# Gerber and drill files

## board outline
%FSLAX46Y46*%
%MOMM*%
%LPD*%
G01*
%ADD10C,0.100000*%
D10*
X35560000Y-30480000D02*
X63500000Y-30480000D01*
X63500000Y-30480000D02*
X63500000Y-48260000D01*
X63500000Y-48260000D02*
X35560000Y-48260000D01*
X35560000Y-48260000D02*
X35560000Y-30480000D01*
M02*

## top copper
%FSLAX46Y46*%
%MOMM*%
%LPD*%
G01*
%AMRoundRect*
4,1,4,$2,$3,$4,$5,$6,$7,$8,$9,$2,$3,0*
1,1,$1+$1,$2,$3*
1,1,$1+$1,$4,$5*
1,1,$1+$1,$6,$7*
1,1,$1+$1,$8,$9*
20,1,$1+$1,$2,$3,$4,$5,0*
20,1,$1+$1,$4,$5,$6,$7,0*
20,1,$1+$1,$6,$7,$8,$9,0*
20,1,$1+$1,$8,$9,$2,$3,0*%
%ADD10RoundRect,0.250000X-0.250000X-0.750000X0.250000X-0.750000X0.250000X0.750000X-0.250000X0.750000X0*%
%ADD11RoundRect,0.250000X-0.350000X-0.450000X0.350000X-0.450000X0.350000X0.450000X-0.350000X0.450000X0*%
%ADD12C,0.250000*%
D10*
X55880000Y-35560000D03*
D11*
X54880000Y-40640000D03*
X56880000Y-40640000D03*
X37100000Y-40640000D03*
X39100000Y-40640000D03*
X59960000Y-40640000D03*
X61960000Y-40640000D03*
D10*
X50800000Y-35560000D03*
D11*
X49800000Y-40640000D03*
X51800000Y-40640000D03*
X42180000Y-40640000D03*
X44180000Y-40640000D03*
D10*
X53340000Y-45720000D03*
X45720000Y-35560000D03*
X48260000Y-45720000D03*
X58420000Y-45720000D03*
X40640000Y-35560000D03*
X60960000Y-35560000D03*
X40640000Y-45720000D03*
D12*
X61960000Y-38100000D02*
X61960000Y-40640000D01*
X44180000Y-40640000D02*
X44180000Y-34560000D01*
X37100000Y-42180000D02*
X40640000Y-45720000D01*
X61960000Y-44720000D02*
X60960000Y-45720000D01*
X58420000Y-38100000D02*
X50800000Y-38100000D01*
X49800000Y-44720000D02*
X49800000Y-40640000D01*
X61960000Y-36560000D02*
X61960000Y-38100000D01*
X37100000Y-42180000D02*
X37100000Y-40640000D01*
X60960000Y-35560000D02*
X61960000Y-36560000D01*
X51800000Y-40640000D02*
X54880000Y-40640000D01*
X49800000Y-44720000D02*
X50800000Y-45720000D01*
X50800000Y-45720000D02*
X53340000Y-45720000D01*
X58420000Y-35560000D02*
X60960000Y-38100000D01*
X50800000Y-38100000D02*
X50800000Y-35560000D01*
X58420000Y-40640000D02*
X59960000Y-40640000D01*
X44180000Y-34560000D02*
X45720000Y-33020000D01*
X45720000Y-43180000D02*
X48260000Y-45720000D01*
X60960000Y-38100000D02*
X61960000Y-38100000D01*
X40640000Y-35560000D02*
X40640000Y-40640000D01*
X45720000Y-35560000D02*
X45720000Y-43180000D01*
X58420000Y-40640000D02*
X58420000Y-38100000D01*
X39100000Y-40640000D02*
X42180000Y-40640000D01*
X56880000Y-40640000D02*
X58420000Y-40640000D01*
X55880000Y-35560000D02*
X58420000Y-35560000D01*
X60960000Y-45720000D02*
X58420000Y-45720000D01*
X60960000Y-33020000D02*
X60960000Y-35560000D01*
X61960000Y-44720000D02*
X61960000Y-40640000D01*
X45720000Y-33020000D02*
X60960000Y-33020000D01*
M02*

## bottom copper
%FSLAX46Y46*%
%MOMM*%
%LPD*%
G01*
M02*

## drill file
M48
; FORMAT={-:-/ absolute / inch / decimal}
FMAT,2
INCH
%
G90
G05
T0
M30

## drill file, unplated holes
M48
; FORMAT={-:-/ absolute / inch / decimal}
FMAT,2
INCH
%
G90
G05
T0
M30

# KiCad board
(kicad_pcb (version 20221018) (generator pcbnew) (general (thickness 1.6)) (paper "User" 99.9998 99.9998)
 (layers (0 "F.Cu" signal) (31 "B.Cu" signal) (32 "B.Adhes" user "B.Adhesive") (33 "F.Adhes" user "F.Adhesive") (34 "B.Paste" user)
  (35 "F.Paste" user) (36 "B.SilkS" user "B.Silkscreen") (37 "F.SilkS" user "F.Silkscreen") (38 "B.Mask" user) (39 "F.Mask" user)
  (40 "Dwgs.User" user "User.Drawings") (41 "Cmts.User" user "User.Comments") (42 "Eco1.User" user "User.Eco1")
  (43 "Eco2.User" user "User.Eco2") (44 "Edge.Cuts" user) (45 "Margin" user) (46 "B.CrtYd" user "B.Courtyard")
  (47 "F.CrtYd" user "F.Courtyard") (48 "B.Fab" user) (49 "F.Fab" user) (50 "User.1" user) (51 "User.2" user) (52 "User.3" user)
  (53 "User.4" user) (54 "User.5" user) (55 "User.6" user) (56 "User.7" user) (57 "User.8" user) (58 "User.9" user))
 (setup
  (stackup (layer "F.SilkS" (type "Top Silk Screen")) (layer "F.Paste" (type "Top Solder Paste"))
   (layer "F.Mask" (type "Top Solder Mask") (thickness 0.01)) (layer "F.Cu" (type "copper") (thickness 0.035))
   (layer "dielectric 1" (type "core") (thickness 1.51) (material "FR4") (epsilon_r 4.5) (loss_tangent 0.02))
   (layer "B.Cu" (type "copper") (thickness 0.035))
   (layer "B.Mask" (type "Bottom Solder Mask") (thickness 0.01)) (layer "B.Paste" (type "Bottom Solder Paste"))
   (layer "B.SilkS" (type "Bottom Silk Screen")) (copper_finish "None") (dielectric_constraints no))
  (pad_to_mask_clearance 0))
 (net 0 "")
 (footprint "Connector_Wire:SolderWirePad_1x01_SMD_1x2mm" (layer "F.Cu") (at 55.88 35.56)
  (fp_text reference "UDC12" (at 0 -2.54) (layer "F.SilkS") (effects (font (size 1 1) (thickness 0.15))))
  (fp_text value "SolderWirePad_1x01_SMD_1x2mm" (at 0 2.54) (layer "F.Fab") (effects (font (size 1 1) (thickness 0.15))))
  (pad "1" smd roundrect (at 0 0) (size 1 2) (layers "F.Cu" "F.Paste" "F.Mask") (roundrect_rratio 0.25)))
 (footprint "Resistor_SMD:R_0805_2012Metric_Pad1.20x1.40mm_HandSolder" (layer "F.Cu") (at 55.88 40.64)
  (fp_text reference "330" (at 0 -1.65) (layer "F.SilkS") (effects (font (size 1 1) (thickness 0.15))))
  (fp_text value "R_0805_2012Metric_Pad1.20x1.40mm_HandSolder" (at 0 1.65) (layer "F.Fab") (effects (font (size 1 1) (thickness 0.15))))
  (pad "1" smd roundrect (at -1 0) (size 1.2 1.4) (layers "F.Cu" "F.Paste" "F.Mask") (roundrect_rratio 0.2083333333))
  (pad "2" smd roundrect (at 1 0) (size 1.2 1.4) (layers "F.Cu" "F.Paste" "F.Mask") (roundrect_rratio 0.2083333333)))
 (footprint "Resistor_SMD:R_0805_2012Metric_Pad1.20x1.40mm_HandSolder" (layer "F.Cu") (at 38.1 40.64)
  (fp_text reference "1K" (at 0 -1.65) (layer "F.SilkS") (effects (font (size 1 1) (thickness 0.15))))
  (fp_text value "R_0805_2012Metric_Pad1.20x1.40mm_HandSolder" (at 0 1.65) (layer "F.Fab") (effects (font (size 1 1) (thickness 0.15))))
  (pad "1" smd roundrect (at -1 0) (size 1.2 1.4) (layers "F.Cu" "F.Paste" "F.Mask") (roundrect_rratio 0.2083333333))
  (pad "2" smd roundrect (at 1 0) (size 1.2 1.4) (layers "F.Cu" "F.Paste" "F.Mask") (roundrect_rratio 0.2083333333)))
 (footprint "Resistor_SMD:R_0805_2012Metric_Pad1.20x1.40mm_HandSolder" (layer "F.Cu") (at 60.96 40.64)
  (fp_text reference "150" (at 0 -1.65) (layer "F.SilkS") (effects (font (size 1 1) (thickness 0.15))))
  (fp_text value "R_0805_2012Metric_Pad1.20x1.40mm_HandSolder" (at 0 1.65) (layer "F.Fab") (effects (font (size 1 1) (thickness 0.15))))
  (pad "1" smd roundrect (at -1 0) (size 1.2 1.4) (layers "F.Cu" "F.Paste" "F.Mask") (roundrect_rratio 0.2083333333))
  (pad "2" smd roundrect (at 1 0) (size 1.2 1.4) (layers "F.Cu" "F.Paste" "F.Mask") (roundrect_rratio 0.2083333333)))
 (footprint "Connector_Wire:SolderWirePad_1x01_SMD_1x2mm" (layer "F.Cu") (at 50.8 35.56)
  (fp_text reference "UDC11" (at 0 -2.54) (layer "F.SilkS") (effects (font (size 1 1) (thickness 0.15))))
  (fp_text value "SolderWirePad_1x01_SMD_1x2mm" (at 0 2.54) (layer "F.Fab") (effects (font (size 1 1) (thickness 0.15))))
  (pad "1" smd roundrect (at 0 0) (size 1 2) (layers "F.Cu" "F.Paste" "F.Mask") (roundrect_rratio 0.25)))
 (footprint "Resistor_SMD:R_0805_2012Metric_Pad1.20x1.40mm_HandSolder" (layer "F.Cu") (at 50.8 40.64)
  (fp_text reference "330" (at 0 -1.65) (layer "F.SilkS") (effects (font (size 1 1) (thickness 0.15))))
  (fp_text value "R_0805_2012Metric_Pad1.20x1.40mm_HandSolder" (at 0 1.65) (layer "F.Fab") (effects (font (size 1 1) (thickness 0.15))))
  (pad "1" smd roundrect (at -1 0) (size 1.2 1.4) (layers "F.Cu" "F.Paste" "F.Mask") (roundrect_rratio 0.2083333333))
  (pad "2" smd roundrect (at 1 0) (size 1.2 1.4) (layers "F.Cu" "F.Paste" "F.Mask") (roundrect_rratio 0.2083333333)))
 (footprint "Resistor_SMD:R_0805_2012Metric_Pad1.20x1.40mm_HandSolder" (layer "F.Cu") (at 43.18 40.64)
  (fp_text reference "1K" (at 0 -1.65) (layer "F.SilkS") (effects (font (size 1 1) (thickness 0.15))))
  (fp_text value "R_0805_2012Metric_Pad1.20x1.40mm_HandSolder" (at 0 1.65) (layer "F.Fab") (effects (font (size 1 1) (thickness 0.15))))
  (pad "1" smd roundrect (at -1 0) (size 1.2 1.4) (layers "F.Cu" "F.Paste" "F.Mask") (roundrect_rratio 0.2083333333))
  (pad "2" smd roundrect (at 1 0) (size 1.2 1.4) (layers "F.Cu" "F.Paste" "F.Mask") (roundrect_rratio 0.2083333333)))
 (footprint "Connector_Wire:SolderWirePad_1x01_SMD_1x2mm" (layer "F.Cu") (at 53.34 45.72)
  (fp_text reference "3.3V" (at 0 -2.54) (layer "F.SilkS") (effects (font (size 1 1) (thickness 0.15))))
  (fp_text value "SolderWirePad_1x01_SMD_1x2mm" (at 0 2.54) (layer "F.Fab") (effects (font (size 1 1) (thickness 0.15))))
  (pad "1" smd roundrect (at 0 0) (size 1 2) (layers "F.Cu" "F.Paste" "F.Mask") (roundrect_rratio 0.25)))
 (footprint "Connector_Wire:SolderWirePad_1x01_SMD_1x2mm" (layer "F.Cu") (at 45.72 35.56)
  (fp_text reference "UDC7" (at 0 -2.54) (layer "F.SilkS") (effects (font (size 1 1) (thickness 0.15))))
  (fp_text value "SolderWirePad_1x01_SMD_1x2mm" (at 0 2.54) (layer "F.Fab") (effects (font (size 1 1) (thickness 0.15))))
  (pad "1" smd roundrect (at 0 0) (size 1 2) (layers "F.Cu" "F.Paste" "F.Mask") (roundrect_rratio 0.25)))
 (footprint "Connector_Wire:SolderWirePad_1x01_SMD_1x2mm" (layer "F.Cu") (at 48.26 45.72)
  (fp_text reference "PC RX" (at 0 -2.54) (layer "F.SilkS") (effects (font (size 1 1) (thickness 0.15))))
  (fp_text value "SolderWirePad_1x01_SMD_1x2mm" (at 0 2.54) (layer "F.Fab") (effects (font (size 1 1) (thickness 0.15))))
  (pad "1" smd roundrect (at 0 0) (size 1 2) (layers "F.Cu" "F.Paste" "F.Mask") (roundrect_rratio 0.25)))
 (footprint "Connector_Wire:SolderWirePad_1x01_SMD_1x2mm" (layer "F.Cu") (at 58.42 45.72)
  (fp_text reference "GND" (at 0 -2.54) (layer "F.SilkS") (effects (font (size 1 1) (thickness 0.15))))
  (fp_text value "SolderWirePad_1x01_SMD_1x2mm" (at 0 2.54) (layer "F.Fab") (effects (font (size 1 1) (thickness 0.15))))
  (pad "1" smd roundrect (at 0 0) (size 1 2) (layers "F.Cu" "F.Paste" "F.Mask") (roundrect_rratio 0.25)))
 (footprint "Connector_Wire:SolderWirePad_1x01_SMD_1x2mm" (layer "F.Cu") (at 40.64 35.56)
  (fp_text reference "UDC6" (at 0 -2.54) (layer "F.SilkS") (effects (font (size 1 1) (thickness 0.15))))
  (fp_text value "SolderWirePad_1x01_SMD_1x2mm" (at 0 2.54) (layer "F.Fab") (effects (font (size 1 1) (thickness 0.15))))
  (pad "1" smd roundrect (at 0 0) (size 1 2) (layers "F.Cu" "F.Paste" "F.Mask") (roundrect_rratio 0.25)))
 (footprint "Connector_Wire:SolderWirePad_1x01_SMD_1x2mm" (layer "F.Cu") (at 60.96 35.56)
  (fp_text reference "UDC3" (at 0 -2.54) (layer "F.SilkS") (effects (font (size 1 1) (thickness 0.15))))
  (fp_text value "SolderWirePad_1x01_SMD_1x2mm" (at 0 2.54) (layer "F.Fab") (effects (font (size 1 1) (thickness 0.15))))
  (pad "1" smd roundrect (at 0 0) (size 1 2) (layers "F.Cu" "F.Paste" "F.Mask") (roundrect_rratio 0.25)))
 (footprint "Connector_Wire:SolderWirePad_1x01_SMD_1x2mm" (layer "F.Cu") (at 40.64 45.72)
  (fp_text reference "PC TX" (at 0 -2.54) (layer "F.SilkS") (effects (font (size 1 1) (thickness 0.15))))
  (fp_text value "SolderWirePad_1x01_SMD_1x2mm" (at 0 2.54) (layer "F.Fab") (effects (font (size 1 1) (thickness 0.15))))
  (pad "1" smd roundrect (at 0 0) (size 1 2) (layers "F.Cu" "F.Paste" "F.Mask") (roundrect_rratio 0.25)))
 (gr_rect (start 35.56 30.48) (end 63.5 48.26) (stroke (width 0.1) (type default)) (fill none) (layer "Edge.Cuts"))
 (segment (start 61.96 38.1) (end 61.96 40.64) (width 0.25) (layer "F.Cu") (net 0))
 (segment (start 44.18 40.64) (end 44.18 34.56) (width 0.25) (layer "F.Cu") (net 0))
 (segment (start 37.1 42.18) (end 40.64 45.72) (width 0.25) (layer "F.Cu") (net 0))
 (segment (start 61.96 44.72) (end 60.96 45.72) (width 0.25) (layer "F.Cu") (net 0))
 (segment (start 58.42 38.1) (end 50.8 38.1) (width 0.25) (layer "F.Cu") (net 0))
 (segment (start 49.8 44.72) (end 49.8 40.64) (width 0.25) (layer "F.Cu") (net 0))
 (segment (start 61.96 36.56) (end 61.96 38.1) (width 0.25) (layer "F.Cu") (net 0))
 (segment (start 37.1 42.18) (end 37.1 40.64) (width 0.25) (layer "F.Cu") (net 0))
 (segment (start 60.96 35.56) (end 61.96 36.56) (width 0.25) (layer "F.Cu") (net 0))
 (segment (start 51.8 40.64) (end 54.88 40.64) (width 0.25) (layer "F.Cu") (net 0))
 (segment (start 49.8 44.72) (end 50.8 45.72) (width 0.25) (layer "F.Cu") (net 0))
 (segment (start 50.8 45.72) (end 53.34 45.72) (width 0.25) (layer "F.Cu") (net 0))
 (segment (start 58.42 35.56) (end 60.96 38.1) (width 0.25) (layer "F.Cu") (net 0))
 (segment (start 50.8 38.1) (end 50.8 35.56) (width 0.25) (layer "F.Cu") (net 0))
 (segment (start 58.42 40.64) (end 59.96 40.64) (width 0.25) (layer "F.Cu") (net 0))
 (segment (start 44.18 34.56) (end 45.72 33.02) (width 0.25) (layer "F.Cu") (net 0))
 (segment (start 45.72 43.18) (end 48.26 45.72) (width 0.25) (layer "F.Cu") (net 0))
 (segment (start 60.96 38.1) (end 61.96 38.1) (width 0.25) (layer "F.Cu") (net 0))
 (segment (start 40.64 35.56) (end 40.64 40.64) (width 0.25) (layer "F.Cu") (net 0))
 (segment (start 45.72 35.56) (end 45.72 43.18) (width 0.25) (layer "F.Cu") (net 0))
 (segment (start 58.42 40.64) (end 58.42 38.1) (width 0.25) (layer "F.Cu") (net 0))
 (segment (start 39.1 40.64) (end 42.18 40.64) (width 0.25) (layer "F.Cu") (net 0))
 (segment (start 56.88 40.64) (end 58.42 40.64) (width 0.25) (layer "F.Cu") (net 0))
 (segment (start 55.88 35.56) (end 58.42 35.56) (width 0.25) (layer "F.Cu") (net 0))
 (segment (start 60.96 45.72) (end 58.42 45.72) (width 0.25) (layer "F.Cu") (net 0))
 (segment (start 60.96 33.02) (end 60.96 35.56) (width 0.25) (layer "F.Cu") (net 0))
 (segment (start 61.96 44.72) (end 61.96 40.64) (width 0.25) (layer "F.Cu") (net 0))
 (segment (start 45.72 33.02) (end 60.96 33.02) (width 0.25) (layer "F.Cu") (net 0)))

